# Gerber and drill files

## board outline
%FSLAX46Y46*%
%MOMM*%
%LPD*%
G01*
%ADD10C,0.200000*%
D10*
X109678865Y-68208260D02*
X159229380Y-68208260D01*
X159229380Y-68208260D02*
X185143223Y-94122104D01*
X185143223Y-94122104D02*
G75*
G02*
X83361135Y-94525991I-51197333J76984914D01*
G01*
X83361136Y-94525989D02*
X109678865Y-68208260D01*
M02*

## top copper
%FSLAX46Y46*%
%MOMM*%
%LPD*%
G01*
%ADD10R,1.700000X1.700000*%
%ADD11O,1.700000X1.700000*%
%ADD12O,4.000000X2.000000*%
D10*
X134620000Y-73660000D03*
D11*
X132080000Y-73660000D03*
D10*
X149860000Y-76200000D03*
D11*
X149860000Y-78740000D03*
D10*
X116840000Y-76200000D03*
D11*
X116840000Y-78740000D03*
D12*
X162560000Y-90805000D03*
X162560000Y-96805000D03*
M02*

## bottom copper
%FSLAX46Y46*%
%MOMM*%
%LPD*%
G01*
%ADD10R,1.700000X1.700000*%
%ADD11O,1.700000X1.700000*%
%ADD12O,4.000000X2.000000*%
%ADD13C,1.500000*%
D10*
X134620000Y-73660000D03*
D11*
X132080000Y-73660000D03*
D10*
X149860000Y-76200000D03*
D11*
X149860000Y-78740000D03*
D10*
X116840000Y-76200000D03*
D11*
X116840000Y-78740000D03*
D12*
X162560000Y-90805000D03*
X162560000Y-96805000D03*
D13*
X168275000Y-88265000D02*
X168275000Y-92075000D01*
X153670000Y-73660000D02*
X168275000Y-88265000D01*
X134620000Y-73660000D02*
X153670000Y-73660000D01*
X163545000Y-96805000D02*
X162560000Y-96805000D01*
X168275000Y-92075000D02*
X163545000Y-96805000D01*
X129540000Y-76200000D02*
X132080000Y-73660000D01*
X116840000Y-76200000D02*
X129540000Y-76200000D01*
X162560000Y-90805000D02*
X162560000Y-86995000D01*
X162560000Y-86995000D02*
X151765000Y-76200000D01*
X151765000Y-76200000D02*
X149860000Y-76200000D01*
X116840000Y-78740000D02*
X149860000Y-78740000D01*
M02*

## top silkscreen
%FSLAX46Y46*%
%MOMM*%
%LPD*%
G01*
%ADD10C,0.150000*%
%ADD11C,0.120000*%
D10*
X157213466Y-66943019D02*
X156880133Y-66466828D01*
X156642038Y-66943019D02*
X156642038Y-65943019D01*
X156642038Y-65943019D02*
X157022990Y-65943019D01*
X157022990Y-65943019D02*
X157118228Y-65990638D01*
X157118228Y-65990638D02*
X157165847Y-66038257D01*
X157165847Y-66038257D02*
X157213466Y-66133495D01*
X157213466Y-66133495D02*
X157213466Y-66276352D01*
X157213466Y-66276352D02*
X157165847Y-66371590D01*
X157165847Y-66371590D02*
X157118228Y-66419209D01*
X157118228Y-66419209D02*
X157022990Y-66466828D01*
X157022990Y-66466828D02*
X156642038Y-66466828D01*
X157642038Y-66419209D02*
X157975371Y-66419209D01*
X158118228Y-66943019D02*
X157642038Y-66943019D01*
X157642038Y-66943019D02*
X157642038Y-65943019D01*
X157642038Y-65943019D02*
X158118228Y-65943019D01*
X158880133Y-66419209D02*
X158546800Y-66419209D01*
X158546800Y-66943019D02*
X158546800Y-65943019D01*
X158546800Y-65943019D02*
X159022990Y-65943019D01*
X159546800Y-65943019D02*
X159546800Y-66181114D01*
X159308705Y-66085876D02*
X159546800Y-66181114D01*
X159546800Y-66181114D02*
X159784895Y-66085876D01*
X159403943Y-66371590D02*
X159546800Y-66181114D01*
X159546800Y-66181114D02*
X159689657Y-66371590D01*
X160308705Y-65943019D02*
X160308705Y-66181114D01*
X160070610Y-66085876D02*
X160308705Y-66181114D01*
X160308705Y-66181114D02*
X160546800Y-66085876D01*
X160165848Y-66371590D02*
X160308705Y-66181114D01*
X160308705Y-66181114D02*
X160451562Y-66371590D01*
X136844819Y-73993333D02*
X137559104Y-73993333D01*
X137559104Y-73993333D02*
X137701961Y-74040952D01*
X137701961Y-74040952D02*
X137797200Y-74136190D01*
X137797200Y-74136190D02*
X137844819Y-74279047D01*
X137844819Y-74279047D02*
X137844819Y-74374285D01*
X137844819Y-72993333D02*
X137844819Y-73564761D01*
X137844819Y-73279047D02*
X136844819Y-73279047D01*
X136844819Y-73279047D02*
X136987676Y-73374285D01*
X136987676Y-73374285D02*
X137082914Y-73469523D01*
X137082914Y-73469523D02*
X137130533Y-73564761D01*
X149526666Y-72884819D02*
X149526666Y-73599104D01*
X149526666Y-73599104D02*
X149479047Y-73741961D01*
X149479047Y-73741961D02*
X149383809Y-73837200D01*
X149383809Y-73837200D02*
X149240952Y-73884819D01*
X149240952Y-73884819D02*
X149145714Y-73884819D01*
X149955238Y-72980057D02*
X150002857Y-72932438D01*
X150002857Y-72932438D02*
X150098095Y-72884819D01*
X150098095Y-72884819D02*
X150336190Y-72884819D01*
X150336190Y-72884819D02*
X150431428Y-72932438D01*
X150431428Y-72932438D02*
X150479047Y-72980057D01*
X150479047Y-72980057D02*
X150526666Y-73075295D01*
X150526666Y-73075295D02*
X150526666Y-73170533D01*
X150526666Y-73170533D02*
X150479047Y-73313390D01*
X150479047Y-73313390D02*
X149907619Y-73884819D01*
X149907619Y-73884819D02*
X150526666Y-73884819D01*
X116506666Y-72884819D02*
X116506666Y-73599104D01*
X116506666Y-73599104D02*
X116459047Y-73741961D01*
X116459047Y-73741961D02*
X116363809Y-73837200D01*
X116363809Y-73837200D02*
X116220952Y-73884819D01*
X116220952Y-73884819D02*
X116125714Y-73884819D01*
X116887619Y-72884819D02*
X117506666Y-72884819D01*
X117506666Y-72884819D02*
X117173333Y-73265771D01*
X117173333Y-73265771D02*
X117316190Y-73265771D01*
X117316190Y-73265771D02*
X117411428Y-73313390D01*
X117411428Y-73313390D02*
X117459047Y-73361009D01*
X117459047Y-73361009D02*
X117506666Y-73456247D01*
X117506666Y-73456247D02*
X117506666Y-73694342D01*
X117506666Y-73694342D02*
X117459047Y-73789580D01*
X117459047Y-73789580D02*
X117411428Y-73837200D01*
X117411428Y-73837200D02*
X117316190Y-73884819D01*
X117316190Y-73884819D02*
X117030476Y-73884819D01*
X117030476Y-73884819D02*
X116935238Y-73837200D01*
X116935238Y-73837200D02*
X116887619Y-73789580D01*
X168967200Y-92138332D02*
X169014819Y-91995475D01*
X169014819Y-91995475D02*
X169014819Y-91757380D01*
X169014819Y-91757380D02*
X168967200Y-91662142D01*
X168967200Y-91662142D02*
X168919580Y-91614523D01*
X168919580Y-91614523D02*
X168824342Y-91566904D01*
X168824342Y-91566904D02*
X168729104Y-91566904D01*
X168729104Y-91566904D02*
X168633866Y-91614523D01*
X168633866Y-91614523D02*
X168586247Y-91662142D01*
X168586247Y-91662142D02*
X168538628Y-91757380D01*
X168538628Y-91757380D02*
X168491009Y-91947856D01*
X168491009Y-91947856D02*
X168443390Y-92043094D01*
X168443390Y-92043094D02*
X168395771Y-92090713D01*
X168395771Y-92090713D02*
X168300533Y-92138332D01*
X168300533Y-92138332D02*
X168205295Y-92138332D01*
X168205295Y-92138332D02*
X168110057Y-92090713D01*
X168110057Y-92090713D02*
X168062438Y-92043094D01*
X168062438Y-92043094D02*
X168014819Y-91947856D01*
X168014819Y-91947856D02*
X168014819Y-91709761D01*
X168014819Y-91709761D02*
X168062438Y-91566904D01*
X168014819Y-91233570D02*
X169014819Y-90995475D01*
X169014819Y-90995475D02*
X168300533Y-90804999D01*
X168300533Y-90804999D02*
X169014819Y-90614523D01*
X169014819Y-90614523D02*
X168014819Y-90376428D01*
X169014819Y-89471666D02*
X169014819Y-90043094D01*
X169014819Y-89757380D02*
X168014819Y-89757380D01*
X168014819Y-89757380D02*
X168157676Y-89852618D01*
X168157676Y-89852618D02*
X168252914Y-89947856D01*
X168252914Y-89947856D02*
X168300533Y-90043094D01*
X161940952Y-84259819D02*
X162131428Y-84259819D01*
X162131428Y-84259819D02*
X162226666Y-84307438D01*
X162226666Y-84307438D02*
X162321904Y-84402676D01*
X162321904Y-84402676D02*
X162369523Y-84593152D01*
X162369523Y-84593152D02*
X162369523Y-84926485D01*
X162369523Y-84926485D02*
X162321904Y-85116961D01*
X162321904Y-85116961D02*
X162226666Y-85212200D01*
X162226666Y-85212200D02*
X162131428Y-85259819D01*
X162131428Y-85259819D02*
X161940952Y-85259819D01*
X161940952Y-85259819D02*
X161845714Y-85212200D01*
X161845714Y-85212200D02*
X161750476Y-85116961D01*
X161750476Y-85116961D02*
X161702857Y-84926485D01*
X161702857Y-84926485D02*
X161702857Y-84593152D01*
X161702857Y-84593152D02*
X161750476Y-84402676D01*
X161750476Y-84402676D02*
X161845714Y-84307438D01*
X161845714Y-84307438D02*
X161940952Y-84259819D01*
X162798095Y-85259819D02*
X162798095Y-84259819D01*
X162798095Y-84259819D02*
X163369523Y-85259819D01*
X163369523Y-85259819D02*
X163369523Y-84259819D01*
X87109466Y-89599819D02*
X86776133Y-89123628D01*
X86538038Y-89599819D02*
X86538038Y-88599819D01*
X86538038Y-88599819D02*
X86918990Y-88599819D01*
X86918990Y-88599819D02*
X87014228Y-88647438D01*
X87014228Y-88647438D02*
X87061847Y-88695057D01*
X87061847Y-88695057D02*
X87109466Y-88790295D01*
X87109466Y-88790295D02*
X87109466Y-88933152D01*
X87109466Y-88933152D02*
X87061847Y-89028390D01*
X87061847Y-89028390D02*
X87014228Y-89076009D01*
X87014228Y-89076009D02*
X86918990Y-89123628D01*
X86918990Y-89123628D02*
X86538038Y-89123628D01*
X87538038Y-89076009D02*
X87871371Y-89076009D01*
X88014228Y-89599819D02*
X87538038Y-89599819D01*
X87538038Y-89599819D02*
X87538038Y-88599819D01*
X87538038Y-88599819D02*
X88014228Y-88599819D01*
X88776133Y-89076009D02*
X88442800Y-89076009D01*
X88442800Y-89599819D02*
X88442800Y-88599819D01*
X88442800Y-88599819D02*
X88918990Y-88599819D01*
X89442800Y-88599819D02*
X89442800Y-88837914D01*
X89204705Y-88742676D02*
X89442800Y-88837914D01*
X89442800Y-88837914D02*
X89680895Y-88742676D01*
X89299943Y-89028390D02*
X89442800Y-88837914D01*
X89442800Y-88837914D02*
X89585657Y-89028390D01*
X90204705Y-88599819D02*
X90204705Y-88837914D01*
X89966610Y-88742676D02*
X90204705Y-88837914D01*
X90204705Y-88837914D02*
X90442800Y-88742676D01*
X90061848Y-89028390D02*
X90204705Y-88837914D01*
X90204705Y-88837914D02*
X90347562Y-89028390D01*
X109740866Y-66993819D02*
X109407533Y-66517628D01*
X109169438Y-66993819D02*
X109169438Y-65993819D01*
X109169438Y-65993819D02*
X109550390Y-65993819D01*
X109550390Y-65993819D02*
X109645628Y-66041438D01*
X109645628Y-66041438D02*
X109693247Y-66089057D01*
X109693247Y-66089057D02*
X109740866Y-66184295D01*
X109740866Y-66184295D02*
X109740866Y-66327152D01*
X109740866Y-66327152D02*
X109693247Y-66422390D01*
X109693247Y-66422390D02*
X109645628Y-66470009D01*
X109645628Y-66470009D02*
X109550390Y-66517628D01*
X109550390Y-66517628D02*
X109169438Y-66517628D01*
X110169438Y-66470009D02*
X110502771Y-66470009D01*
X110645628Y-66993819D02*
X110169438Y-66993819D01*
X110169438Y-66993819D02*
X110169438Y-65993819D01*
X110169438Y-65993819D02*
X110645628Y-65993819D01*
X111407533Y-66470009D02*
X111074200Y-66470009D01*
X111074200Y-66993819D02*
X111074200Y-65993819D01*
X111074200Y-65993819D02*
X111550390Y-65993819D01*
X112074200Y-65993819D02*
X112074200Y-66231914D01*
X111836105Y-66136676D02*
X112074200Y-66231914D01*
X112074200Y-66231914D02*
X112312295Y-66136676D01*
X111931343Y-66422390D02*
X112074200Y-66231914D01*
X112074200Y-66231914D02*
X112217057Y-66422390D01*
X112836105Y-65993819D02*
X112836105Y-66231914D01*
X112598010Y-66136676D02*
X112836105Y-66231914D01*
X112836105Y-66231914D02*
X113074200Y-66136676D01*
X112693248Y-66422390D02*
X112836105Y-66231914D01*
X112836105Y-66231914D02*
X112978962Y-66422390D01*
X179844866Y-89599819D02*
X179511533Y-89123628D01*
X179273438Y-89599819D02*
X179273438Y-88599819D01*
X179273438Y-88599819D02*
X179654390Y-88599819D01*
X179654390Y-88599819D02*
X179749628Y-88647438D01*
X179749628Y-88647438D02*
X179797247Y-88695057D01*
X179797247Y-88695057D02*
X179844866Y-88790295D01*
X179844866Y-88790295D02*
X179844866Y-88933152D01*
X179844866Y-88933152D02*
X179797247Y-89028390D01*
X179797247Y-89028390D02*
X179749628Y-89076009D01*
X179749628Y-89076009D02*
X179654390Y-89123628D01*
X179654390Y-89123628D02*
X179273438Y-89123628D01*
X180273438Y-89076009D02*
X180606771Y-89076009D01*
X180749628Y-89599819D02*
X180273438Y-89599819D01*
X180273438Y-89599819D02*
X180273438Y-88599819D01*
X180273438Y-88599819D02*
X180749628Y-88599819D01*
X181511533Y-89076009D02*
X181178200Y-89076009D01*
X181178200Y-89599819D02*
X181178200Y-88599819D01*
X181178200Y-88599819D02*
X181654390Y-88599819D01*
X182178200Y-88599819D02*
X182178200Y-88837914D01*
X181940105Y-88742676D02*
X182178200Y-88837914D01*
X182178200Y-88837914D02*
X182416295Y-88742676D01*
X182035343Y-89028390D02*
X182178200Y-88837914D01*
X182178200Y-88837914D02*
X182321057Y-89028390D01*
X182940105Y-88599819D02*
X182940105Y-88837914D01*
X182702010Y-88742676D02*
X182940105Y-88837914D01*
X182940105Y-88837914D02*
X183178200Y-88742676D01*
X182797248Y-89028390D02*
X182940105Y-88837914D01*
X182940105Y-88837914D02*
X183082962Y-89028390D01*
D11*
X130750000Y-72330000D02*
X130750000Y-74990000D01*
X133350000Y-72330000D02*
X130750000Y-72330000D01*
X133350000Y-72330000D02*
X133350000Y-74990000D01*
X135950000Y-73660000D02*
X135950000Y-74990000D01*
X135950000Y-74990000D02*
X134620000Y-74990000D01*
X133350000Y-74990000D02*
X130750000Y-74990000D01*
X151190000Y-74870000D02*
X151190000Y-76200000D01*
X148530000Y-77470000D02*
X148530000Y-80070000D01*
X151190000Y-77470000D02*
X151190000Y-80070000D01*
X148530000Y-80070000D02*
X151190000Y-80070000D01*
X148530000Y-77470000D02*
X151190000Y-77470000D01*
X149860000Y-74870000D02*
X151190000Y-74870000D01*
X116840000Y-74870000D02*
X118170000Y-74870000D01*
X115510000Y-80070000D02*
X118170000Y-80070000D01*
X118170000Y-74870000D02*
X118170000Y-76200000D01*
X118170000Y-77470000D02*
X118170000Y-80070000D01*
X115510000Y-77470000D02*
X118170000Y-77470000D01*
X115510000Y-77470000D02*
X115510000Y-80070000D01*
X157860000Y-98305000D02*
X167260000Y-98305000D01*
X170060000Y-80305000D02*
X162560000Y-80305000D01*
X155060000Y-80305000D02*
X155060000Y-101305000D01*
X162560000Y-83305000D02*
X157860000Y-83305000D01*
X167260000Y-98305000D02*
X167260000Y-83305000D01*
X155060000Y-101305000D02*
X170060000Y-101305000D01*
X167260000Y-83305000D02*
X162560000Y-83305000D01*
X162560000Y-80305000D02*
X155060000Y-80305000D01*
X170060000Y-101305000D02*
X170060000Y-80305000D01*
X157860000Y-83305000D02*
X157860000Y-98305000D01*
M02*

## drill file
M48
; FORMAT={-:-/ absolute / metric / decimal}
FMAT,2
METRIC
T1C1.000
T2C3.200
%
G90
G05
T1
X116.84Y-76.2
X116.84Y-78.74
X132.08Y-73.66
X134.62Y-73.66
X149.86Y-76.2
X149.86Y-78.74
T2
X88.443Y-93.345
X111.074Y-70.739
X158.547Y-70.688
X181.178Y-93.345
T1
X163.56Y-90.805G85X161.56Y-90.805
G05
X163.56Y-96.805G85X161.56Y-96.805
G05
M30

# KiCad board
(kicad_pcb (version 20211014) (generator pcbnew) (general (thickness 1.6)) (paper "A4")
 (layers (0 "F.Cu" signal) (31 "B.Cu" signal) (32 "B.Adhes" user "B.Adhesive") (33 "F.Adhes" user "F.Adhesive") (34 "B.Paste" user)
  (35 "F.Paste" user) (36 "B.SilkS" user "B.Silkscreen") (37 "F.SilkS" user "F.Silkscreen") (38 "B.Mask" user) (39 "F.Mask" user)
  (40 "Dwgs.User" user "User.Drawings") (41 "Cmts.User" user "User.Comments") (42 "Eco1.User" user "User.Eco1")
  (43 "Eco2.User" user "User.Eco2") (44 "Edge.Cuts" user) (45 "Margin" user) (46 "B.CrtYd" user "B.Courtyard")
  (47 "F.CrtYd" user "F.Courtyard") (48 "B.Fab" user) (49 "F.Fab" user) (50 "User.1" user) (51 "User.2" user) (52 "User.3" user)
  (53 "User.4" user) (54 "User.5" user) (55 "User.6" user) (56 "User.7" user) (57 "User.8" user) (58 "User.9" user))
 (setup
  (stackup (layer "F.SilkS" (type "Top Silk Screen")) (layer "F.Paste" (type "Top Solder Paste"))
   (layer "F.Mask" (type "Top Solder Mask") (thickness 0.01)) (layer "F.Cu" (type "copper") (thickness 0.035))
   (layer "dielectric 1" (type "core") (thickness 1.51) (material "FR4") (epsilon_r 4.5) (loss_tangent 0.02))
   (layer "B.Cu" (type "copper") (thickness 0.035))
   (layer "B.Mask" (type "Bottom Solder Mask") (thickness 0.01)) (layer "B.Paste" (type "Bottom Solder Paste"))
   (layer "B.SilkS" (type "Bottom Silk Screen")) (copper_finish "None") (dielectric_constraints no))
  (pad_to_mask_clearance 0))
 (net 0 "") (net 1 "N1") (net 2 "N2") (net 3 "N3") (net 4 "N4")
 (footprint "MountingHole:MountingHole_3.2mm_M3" (layer "F.Cu") (at 158.5468 70.6882)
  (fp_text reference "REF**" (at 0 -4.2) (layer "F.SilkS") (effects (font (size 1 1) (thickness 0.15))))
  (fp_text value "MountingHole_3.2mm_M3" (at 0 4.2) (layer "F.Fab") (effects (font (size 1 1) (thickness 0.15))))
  (pad "" np_thru_hole circle (at 0 0) (size 3.2 3.2) (drill 3.2) (layers *.Cu *.Mask)))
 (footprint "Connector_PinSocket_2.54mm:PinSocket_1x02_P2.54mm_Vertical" (layer "F.Cu") (at 134.62 73.66 -90)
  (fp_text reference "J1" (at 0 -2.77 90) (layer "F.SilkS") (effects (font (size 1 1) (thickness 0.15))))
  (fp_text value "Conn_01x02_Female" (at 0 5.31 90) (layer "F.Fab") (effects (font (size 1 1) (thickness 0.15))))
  (fp_line (start -1.33 3.87) (end 1.33 3.87) (layer "F.SilkS") (width 0.12))
  (fp_line (start -1.33 1.27) (end -1.33 3.87) (layer "F.SilkS") (width 0.12))
  (fp_line (start -1.33 1.27) (end 1.33 1.27) (layer "F.SilkS") (width 0.12))
  (fp_line (start 0 -1.33) (end 1.33 -1.33) (layer "F.SilkS") (width 0.12))
  (fp_line (start 1.33 -1.33) (end 1.33 0) (layer "F.SilkS") (width 0.12))
  (fp_line (start 1.33 1.27) (end 1.33 3.87) (layer "F.SilkS") (width 0.12))
  (pad "1" thru_hole rect (at 0 0 270) (size 1.7 1.7) (drill 1) (layers *.Cu *.Mask) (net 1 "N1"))
  (pad "2" thru_hole oval (at 0 2.54 270) (size 1.7 1.7) (drill 1) (layers *.Cu *.Mask) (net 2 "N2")))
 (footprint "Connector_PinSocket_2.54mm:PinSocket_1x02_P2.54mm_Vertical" (layer "F.Cu") (at 149.86 76.2)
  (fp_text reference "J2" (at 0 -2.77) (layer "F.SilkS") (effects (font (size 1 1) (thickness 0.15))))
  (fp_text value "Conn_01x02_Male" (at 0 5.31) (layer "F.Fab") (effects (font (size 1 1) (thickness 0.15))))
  (fp_line (start 1.33 -1.33) (end 1.33 0) (layer "F.SilkS") (width 0.12))
  (fp_line (start -1.33 1.27) (end -1.33 3.87) (layer "F.SilkS") (width 0.12))
  (fp_line (start 1.33 1.27) (end 1.33 3.87) (layer "F.SilkS") (width 0.12))
  (fp_line (start -1.33 3.87) (end 1.33 3.87) (layer "F.SilkS") (width 0.12))
  (fp_line (start -1.33 1.27) (end 1.33 1.27) (layer "F.SilkS") (width 0.12))
  (fp_line (start 0 -1.33) (end 1.33 -1.33) (layer "F.SilkS") (width 0.12))
  (pad "1" thru_hole rect (at 0 0) (size 1.7 1.7) (drill 1) (layers *.Cu *.Mask) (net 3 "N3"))
  (pad "2" thru_hole oval (at 0 2.54) (size 1.7 1.7) (drill 1) (layers *.Cu *.Mask) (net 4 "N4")))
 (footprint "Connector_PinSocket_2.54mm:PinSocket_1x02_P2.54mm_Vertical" (layer "F.Cu") (at 116.84 76.2)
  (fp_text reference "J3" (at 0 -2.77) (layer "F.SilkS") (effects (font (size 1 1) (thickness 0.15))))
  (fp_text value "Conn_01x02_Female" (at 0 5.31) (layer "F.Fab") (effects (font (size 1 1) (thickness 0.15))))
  (fp_line (start 0 -1.33) (end 1.33 -1.33) (layer "F.SilkS") (width 0.12))
  (fp_line (start -1.33 3.87) (end 1.33 3.87) (layer "F.SilkS") (width 0.12))
  (fp_line (start 1.33 -1.33) (end 1.33 0) (layer "F.SilkS") (width 0.12))
  (fp_line (start 1.33 1.27) (end 1.33 3.87) (layer "F.SilkS") (width 0.12))
  (fp_line (start -1.33 1.27) (end 1.33 1.27) (layer "F.SilkS") (width 0.12))
  (fp_line (start -1.33 1.27) (end -1.33 3.87) (layer "F.SilkS") (width 0.12))
  (pad "1" thru_hole rect (at 0 0) (size 1.7 1.7) (drill 1) (layers *.Cu *.Mask) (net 2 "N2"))
  (pad "2" thru_hole oval (at 0 2.54) (size 1.7 1.7) (drill 1) (layers *.Cu *.Mask) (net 4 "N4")))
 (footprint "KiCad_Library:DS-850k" (layer "F.Cu") (at 162.56 90.805 90)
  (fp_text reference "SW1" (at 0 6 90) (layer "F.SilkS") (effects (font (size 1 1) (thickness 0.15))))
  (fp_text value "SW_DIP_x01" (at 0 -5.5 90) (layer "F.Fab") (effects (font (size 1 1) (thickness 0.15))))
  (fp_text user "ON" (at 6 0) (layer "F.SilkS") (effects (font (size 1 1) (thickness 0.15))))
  (fp_line (start -7.5 -4.7) (end -7.5 4.7) (layer "F.SilkS") (width 0.12))
  (fp_line (start 10.5 7.5) (end 10.5 0) (layer "F.SilkS") (width 0.12))
  (fp_line (start 10.5 -7.5) (end -10.5 -7.5) (layer "F.SilkS") (width 0.12))
  (fp_line (start 7.5 0) (end 7.5 -4.7) (layer "F.SilkS") (width 0.12))
  (fp_line (start -7.5 4.7) (end 7.5 4.7) (layer "F.SilkS") (width 0.12))
  (fp_line (start -10.5 -7.5) (end -10.5 7.5) (layer "F.SilkS") (width 0.12))
  (fp_line (start 7.5 4.7) (end 7.5 0) (layer "F.SilkS") (width 0.12))
  (fp_line (start 10.5 0) (end 10.5 -7.5) (layer "F.SilkS") (width 0.12))
  (fp_line (start -10.5 7.5) (end 10.5 7.5) (layer "F.SilkS") (width 0.12))
  (fp_line (start 7.5 -4.7) (end -7.5 -4.7) (layer "F.SilkS") (width 0.12))
  (pad "1" thru_hole oval locked (at 0 0 180) (size 4 2) (drill oval 3 1) (layers *.Cu *.Mask) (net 3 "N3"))
  (pad "2" thru_hole oval locked (at -6 0 180) (size 4 2) (drill oval 3 1) (layers *.Cu *.Mask) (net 1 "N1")))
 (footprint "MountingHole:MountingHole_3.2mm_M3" (layer "F.Cu") (at 88.4428 93.345)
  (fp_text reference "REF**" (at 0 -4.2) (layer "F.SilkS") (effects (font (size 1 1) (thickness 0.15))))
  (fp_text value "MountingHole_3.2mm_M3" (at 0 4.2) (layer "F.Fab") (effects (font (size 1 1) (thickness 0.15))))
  (pad "" np_thru_hole circle (at 0 0) (size 3.2 3.2) (drill 3.2) (layers *.Cu *.Mask)))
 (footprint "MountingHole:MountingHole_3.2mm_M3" (layer "F.Cu") (at 111.0742 70.739)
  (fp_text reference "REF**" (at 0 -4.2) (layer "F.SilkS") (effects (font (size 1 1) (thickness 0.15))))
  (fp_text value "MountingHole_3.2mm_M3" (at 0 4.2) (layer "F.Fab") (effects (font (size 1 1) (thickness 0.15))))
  (pad "" np_thru_hole circle (at 0 0) (size 3.2 3.2) (drill 3.2) (layers *.Cu *.Mask)))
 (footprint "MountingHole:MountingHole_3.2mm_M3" (layer "F.Cu") (at 181.1782 93.345)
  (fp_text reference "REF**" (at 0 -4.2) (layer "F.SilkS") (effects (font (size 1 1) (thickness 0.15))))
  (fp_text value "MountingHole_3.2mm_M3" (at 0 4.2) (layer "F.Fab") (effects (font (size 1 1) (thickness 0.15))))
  (pad "" np_thru_hole circle (at 0 0) (size 3.2 3.2) (drill 3.2) (layers *.Cu *.Mask)))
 (gr_line (start 109.678865 68.20826) (end 159.22938 68.20826) (layer "Edge.Cuts") (width 0.2))
 (gr_line (start 159.22938 68.20826) (end 185.143223 94.122104) (layer "Edge.Cuts") (width 0.2))
 (gr_arc (start 185.143223 94.122104) (mid 134.312761 109.591012) (end 83.361136 94.525989) (layer "Edge.Cuts") (width 0.2))
 (gr_line (start 83.361136 94.525989) (end 109.678865 68.20826) (layer "Edge.Cuts") (width 0.2))
 (segment (start 168.275 88.265) (end 168.275 92.075) (width 1.5) (layer "B.Cu") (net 1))
 (segment (start 153.67 73.66) (end 168.275 88.265) (width 1.5) (layer "B.Cu") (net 1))
 (segment (start 134.62 73.66) (end 153.67 73.66) (width 1.5) (layer "B.Cu") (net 1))
 (segment (start 163.545 96.805) (end 162.56 96.805) (width 1.5) (layer "B.Cu") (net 1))
 (segment (start 168.275 92.075) (end 163.545 96.805) (width 1.5) (layer "B.Cu") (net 1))
 (segment (start 129.54 76.2) (end 132.08 73.66) (width 1.5) (layer "B.Cu") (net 2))
 (segment (start 116.84 76.2) (end 129.54 76.2) (width 1.5) (layer "B.Cu") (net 2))
 (segment (start 162.56 90.805) (end 162.56 86.995) (width 1.5) (layer "B.Cu") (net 3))
 (segment (start 162.56 86.995) (end 151.765 76.2) (width 1.5) (layer "B.Cu") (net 3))
 (segment (start 151.765 76.2) (end 149.86 76.2) (width 1.5) (layer "B.Cu") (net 3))
 (segment (start 116.84 78.74) (end 149.86 78.74) (width 1.5) (layer "B.Cu") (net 4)))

